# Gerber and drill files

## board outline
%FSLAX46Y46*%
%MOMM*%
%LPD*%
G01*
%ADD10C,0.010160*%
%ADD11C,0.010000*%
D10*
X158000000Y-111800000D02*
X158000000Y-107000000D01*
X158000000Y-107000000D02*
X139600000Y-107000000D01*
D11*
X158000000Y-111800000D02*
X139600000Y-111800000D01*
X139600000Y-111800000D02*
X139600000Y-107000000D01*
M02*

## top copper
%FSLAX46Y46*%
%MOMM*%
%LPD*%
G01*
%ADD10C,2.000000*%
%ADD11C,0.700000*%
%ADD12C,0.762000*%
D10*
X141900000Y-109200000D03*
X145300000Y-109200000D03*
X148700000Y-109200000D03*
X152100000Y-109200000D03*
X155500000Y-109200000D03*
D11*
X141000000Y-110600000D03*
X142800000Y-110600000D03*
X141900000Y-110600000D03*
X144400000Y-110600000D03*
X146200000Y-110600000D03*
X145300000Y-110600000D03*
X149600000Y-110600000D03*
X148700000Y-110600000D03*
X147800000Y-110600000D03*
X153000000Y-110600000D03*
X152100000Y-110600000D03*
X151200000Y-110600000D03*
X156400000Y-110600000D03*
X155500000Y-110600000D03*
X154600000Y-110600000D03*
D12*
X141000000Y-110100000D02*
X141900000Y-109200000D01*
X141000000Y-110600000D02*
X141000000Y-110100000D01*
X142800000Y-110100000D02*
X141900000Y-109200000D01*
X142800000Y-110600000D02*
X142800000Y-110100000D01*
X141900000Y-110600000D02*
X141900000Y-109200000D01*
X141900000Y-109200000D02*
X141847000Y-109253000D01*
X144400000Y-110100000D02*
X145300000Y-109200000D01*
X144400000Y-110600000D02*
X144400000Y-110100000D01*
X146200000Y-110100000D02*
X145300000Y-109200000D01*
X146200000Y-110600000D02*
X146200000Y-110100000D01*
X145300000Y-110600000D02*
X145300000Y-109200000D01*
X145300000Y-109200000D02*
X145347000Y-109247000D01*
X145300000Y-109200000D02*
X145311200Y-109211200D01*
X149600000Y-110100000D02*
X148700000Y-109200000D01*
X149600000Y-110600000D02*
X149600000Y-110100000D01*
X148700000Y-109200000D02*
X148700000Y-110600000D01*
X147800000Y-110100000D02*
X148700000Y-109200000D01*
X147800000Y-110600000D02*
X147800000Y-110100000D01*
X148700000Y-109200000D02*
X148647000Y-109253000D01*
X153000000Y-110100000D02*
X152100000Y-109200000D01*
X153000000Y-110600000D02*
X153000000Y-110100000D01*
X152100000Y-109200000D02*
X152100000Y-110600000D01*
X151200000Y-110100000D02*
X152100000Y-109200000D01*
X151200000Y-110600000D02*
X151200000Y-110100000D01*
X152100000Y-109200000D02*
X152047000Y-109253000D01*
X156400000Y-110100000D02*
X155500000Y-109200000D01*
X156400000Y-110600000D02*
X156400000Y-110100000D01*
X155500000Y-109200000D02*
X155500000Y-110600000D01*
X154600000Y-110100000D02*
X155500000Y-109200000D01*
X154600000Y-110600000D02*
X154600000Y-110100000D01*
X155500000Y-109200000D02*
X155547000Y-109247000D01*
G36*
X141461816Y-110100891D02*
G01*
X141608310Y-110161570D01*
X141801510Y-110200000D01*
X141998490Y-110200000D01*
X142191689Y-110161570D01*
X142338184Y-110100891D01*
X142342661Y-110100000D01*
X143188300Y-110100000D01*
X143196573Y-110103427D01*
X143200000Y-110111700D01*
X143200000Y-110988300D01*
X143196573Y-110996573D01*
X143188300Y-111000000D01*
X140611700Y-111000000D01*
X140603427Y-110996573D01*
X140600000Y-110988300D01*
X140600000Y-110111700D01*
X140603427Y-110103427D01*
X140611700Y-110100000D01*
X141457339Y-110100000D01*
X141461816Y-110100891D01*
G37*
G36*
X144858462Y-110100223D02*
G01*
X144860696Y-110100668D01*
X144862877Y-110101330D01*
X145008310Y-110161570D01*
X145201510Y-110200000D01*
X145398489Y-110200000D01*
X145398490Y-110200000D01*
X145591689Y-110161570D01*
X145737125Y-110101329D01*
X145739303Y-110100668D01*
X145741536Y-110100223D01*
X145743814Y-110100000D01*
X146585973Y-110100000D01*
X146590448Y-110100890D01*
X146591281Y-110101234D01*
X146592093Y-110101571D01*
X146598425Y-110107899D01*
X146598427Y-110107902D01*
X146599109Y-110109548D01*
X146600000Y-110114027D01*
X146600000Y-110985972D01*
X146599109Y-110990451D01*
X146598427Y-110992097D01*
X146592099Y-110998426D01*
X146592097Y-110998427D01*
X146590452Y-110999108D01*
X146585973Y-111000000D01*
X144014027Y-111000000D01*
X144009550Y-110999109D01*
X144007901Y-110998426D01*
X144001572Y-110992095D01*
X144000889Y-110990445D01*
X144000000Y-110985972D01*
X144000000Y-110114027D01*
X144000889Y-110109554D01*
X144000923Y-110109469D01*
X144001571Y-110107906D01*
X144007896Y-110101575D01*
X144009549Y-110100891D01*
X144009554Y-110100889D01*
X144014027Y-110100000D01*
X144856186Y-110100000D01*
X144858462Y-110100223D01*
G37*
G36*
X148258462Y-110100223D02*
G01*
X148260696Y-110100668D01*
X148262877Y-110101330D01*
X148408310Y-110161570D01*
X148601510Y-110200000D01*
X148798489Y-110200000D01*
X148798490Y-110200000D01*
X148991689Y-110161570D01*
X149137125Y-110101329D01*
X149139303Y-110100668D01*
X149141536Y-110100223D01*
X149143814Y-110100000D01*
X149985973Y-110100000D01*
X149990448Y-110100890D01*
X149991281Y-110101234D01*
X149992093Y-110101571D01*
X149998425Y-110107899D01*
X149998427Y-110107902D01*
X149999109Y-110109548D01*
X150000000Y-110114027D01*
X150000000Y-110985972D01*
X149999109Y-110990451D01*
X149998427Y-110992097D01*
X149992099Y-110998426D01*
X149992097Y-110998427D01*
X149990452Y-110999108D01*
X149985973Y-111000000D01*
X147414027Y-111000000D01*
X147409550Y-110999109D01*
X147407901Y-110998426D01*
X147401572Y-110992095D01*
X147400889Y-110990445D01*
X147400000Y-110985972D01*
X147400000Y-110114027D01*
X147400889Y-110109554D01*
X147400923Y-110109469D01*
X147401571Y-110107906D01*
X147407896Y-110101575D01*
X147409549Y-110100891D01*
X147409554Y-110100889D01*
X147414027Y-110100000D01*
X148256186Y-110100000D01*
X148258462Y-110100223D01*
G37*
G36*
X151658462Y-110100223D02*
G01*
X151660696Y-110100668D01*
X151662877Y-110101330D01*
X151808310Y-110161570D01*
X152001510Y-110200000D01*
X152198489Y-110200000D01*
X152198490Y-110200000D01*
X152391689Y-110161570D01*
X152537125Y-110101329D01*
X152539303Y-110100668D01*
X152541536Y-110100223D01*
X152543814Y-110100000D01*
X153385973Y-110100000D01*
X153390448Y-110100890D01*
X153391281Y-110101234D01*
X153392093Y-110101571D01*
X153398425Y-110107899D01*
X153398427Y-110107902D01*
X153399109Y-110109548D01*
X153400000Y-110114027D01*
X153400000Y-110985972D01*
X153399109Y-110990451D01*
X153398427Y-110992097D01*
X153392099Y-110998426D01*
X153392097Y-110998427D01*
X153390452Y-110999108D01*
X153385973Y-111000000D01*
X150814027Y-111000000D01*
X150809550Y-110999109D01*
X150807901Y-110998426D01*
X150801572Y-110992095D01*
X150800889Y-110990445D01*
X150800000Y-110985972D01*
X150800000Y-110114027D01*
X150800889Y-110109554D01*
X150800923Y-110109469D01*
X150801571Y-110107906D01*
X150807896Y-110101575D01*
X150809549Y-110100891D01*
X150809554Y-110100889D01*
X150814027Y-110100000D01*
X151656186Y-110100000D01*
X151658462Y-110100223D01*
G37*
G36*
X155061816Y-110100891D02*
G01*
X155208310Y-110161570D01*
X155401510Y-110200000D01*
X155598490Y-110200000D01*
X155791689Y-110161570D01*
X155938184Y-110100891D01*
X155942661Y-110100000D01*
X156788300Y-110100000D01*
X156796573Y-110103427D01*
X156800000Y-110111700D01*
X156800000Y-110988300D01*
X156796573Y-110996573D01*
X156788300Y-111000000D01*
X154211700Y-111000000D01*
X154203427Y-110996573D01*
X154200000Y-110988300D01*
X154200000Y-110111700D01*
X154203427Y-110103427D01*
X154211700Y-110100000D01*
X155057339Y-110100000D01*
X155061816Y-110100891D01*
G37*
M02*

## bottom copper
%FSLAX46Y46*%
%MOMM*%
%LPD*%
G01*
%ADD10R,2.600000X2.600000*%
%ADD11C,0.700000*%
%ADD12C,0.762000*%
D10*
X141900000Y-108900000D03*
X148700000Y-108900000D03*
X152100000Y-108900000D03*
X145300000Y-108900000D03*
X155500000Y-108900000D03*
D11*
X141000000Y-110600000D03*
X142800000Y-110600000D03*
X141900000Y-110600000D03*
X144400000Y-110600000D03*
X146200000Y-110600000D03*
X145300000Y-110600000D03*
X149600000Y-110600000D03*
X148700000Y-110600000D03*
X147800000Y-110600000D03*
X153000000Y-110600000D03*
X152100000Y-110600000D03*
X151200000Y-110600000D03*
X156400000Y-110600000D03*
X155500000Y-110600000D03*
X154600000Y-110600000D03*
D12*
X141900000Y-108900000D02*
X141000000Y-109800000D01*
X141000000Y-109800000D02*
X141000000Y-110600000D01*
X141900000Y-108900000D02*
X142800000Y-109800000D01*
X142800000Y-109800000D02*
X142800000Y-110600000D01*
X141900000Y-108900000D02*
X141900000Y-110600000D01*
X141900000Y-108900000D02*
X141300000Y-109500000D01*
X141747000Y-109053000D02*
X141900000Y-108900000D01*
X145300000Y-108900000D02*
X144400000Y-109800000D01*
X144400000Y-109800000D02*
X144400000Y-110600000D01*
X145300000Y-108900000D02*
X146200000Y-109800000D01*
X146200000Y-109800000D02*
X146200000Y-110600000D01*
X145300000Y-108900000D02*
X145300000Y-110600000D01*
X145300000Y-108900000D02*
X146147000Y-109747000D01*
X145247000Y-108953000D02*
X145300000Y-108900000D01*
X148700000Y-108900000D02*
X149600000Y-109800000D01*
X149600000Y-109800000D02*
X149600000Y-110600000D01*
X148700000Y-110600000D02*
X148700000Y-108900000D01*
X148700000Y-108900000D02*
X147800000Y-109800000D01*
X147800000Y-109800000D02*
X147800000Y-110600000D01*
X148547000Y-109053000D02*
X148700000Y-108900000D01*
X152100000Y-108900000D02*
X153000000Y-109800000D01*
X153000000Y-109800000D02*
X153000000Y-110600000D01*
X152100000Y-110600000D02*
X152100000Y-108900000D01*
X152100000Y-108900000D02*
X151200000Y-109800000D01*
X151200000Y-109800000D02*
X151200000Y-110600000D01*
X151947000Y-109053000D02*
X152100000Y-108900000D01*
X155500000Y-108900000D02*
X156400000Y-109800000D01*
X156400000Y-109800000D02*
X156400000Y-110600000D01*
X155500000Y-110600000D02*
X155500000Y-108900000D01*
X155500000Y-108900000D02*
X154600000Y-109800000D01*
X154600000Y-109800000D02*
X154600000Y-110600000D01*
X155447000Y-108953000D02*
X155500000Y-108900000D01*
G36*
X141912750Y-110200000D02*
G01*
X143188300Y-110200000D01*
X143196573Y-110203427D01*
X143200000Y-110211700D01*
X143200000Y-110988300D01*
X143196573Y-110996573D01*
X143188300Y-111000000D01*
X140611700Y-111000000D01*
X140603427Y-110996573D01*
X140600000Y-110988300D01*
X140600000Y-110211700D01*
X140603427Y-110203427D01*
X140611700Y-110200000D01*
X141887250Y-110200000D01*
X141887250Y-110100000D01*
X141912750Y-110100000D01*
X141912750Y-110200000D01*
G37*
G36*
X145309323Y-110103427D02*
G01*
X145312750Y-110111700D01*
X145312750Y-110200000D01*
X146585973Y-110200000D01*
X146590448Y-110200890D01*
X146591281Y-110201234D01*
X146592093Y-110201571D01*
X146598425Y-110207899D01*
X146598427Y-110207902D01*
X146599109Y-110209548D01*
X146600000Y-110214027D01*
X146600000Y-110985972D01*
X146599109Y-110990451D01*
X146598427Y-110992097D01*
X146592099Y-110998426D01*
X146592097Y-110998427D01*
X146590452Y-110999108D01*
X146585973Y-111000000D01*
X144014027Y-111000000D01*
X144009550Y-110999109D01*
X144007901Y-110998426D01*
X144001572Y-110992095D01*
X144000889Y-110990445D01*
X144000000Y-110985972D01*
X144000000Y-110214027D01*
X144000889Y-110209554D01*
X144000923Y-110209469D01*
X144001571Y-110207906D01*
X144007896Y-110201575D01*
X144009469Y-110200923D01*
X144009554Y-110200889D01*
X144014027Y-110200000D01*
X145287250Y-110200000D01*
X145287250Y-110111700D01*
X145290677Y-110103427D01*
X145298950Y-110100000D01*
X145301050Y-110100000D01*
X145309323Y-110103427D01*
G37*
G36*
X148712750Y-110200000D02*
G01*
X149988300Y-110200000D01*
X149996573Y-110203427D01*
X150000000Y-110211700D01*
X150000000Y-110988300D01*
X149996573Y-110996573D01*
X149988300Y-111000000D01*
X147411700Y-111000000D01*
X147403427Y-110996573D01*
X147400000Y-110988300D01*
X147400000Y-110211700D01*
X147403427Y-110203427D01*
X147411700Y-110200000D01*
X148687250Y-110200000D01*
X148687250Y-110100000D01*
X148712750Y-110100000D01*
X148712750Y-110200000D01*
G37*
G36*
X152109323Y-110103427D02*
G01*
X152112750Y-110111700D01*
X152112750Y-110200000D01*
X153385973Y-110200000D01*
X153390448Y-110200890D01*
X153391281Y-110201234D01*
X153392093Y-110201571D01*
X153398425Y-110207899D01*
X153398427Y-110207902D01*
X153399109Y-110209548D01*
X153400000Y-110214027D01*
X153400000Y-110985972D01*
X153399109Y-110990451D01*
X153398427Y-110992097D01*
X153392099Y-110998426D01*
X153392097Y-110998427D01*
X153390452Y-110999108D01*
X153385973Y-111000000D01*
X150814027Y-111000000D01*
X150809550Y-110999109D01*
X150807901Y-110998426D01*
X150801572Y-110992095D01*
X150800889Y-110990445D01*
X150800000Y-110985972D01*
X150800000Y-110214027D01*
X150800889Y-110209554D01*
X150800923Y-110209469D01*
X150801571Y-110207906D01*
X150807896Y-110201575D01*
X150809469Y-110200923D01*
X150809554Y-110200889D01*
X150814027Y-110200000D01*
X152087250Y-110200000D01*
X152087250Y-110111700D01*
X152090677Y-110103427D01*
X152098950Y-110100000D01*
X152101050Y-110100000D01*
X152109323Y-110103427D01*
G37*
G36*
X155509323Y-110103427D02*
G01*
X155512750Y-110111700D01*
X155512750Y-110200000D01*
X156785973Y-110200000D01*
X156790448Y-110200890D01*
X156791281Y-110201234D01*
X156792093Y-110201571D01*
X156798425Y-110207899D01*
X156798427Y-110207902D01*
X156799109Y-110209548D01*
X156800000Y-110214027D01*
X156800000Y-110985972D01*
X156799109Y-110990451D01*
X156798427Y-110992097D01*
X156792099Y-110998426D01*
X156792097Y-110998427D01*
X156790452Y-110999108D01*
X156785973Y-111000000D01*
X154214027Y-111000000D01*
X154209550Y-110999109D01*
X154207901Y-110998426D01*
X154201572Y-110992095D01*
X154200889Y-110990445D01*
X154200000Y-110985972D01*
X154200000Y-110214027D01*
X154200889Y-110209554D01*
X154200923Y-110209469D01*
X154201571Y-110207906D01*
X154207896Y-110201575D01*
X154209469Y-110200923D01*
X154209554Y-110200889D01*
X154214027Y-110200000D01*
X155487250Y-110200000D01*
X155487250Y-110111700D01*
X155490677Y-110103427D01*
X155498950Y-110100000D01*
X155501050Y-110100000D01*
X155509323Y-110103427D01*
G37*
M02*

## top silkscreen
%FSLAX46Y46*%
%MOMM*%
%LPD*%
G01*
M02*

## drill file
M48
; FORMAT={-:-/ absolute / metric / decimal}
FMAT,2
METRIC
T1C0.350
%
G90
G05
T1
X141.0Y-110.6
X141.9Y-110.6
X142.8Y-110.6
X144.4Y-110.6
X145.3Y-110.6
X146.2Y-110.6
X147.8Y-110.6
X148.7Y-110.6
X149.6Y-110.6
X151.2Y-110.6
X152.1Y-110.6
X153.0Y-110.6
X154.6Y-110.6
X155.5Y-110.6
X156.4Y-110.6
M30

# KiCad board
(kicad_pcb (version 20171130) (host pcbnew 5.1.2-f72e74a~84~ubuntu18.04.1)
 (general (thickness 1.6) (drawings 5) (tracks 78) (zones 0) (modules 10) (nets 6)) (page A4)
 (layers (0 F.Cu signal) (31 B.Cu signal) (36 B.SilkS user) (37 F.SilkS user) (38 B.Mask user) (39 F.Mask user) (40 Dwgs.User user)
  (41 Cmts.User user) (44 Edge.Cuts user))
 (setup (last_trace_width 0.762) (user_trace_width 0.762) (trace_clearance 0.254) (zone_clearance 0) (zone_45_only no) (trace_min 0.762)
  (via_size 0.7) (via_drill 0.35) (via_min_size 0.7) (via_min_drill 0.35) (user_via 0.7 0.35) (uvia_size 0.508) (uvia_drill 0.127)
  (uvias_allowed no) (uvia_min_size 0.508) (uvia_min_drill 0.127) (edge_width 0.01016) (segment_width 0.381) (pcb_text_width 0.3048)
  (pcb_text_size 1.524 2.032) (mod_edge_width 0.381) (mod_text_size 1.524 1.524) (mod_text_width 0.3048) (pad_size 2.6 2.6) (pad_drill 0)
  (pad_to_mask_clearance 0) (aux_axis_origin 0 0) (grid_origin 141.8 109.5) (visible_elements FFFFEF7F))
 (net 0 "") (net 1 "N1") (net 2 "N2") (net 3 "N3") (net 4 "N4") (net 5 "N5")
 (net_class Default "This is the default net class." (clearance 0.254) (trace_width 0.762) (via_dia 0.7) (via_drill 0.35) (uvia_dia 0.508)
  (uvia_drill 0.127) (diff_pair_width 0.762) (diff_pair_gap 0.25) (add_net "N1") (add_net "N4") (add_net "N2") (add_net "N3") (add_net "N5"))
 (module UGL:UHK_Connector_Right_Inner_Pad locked (layer B.Cu) (at 146.31 108.9)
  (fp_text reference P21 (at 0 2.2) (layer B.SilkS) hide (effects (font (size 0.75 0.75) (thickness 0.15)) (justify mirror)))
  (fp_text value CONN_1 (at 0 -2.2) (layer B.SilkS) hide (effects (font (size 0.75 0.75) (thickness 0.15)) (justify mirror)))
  (pad 1 smd rect (at -4.41 0) (size 2.6 2.6) (layers B.Cu B.Mask) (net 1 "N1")))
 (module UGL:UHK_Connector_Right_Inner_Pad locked (layer B.Cu) (at 151.15 108.9)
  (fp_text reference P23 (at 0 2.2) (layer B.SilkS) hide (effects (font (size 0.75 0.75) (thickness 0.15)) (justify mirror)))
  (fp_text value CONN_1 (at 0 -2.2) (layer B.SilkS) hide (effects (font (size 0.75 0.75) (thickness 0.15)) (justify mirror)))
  (pad 1 smd rect (at -2.45 0) (size 2.6 2.6) (layers B.Cu B.Mask) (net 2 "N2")))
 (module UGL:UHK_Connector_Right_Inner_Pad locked (layer B.Cu) (at 153.57 108.9)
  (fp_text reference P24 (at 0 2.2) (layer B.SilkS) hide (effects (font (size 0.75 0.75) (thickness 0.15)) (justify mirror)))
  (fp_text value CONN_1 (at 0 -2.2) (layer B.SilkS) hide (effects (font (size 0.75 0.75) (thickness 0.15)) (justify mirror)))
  (pad 1 smd rect (at -1.47 0) (size 2.6 2.6) (layers B.Cu B.Mask) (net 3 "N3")))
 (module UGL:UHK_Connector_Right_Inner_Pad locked (layer B.Cu) (at 148.73 108.9)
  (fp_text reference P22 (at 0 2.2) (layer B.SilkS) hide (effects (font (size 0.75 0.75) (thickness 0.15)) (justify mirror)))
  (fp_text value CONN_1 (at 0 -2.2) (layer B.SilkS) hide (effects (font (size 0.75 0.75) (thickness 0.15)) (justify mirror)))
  (pad 1 smd rect (at -3.43 0) (size 2.6 2.6) (layers B.Cu B.Mask) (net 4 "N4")))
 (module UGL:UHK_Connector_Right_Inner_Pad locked (layer B.Cu) (at 155.99 108.9)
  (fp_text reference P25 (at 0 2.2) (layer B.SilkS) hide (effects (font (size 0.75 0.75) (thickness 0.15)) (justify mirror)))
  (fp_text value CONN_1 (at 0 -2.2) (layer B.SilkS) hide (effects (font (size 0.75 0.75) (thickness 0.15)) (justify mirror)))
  (pad 1 smd rect (at -0.49 0) (size 2.6 2.6) (layers B.Cu B.Mask) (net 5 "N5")))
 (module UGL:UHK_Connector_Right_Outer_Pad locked (layer F.Cu) (at 141.9 109.2)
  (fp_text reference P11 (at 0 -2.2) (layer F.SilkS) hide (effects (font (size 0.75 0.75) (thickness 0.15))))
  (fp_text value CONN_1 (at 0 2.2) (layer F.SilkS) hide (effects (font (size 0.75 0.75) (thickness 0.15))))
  (pad 1 smd circle (at 0 0) (size 2 2) (layers F.Cu F.Mask) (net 1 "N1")))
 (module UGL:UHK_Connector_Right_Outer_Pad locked (layer F.Cu) (at 145.3 109.2)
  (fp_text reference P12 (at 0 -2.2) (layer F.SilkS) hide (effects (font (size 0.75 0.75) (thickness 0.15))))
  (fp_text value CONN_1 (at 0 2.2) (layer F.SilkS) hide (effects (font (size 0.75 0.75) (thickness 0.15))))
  (pad 1 smd circle (at 0 0) (size 2 2) (layers F.Cu F.Mask) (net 4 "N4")))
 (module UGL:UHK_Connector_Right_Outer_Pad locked (layer F.Cu) (at 148.7 109.2)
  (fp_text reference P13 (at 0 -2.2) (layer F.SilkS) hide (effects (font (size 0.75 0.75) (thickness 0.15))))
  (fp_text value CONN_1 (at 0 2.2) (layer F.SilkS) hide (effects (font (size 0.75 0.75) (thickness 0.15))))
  (pad 1 smd circle (at 0 0) (size 2 2) (layers F.Cu F.Mask) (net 2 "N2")))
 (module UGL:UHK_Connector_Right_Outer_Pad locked (layer F.Cu) (at 152.1 109.2)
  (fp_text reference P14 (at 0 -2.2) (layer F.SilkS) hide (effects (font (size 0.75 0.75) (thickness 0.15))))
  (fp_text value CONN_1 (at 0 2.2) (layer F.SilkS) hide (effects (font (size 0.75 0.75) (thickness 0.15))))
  (pad 1 smd circle (at 0 0) (size 2 2) (layers F.Cu F.Mask) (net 3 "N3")))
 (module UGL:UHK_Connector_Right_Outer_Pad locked (layer F.Cu) (at 155.5 109.2)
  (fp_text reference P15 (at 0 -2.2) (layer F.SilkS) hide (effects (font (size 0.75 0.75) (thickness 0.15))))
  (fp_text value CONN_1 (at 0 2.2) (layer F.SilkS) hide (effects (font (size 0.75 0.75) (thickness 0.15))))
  (pad 1 smd circle (at 0 0) (size 2 2) (layers F.Cu F.Mask) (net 5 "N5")))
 (gr_line (start 158 111.8) (end 158 107) (layer Edge.Cuts) (width 0.01016))
 (gr_line (start 158 107) (end 139.6 107) (layer Edge.Cuts) (width 0.01016))
 (gr_line (start 158 111.8) (end 139.6 111.8) (angle 90) (layer Edge.Cuts) (width 0.01))
 (gr_line (start 139.6 111.8) (end 139.6 107) (angle 90) (layer Edge.Cuts) (width 0.01))
 (segment (start 141.9 108.9) (end 141 109.8) (width 0.762) (layer B.Cu) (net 1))
 (segment (start 141 109.8) (end 141 110.6) (width 0.762) (layer B.Cu) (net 1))
 (segment (start 141 110.1) (end 141.9 109.2) (width 0.762) (layer F.Cu) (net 1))
 (segment (start 141 110.6) (end 141 110.1) (width 0.762) (layer F.Cu) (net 1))
 (via (at 141 110.6) (size 0.7) (drill 0.35) (layers F.Cu B.Cu) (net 1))
 (segment (start 141.9 108.9) (end 142.8 109.8) (width 0.762) (layer B.Cu) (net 1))
 (segment (start 142.8 109.8) (end 142.8 110.6) (width 0.762) (layer B.Cu) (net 1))
 (segment (start 142.8 110.1) (end 141.9 109.2) (width 0.762) (layer F.Cu) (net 1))
 (segment (start 142.8 110.6) (end 142.8 110.1) (width 0.762) (layer F.Cu) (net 1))
 (via (at 142.8 110.6) (size 0.7) (drill 0.35) (layers F.Cu B.Cu) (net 1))
 (segment (start 141.9 108.9) (end 141.9 110.6) (width 0.762) (layer B.Cu) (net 1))
 (segment (start 141.9 110.6) (end 141.9 109.2) (width 0.762) (layer F.Cu) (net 1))
 (via (at 141.9 110.6) (size 0.7) (drill 0.35) (layers F.Cu B.Cu) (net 1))
 (segment (start 141.9 108.9) (end 141.3 109.5) (width 0.762) (layer B.Cu) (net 1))
 (segment (start 141.9 109.2) (end 141.847 109.253) (width 0.762) (layer F.Cu) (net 1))
 (segment (start 141.747 109.053) (end 141.9 108.9) (width 0.762) (layer B.Cu) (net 1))
 (segment (start 145.3 108.9) (end 144.4 109.8) (width 0.762) (layer B.Cu) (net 4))
 (segment (start 144.4 109.8) (end 144.4 110.6) (width 0.762) (layer B.Cu) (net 4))
 (segment (start 144.4 110.1) (end 145.3 109.2) (width 0.762) (layer F.Cu) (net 4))
 (segment (start 144.4 110.6) (end 144.4 110.1) (width 0.762) (layer F.Cu) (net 4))
 (via (at 144.4 110.6) (size 0.7) (drill 0.35) (layers F.Cu B.Cu) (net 4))
 (segment (start 145.3 108.9) (end 146.2 109.8) (width 0.762) (layer B.Cu) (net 4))
 (segment (start 146.2 109.8) (end 146.2 110.6) (width 0.762) (layer B.Cu) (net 4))
 (segment (start 146.2 110.1) (end 145.3 109.2) (width 0.762) (layer F.Cu) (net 4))
 (segment (start 146.2 110.6) (end 146.2 110.1) (width 0.762) (layer F.Cu) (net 4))
 (via (at 146.2 110.6) (size 0.7) (drill 0.35) (layers F.Cu B.Cu) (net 4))
 (segment (start 145.3 108.9) (end 145.3 110.6) (width 0.762) (layer B.Cu) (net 4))
 (segment (start 145.3 110.6) (end 145.3 109.2) (width 0.762) (layer F.Cu) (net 4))
 (via (at 145.3 110.6) (size 0.7) (drill 0.35) (layers F.Cu B.Cu) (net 4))
 (segment (start 145.3 108.9) (end 146.147 109.747) (width 0.762) (layer B.Cu) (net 4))
 (segment (start 145.3 109.2) (end 145.347 109.247) (width 0.762) (layer F.Cu) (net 4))
 (segment (start 145.247 108.953) (end 145.3 108.9) (width 0.762) (layer B.Cu) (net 4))
 (segment (start 145.3 109.2) (end 145.3112 109.2112) (width 0.762) (layer F.Cu) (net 4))
 (segment (start 148.7 108.9) (end 149.6 109.8) (width 0.762) (layer B.Cu) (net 2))
 (segment (start 149.6 109.8) (end 149.6 110.6) (width 0.762) (layer B.Cu) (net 2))
 (segment (start 149.6 110.1) (end 148.7 109.2) (width 0.762) (layer F.Cu) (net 2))
 (segment (start 149.6 110.6) (end 149.6 110.1) (width 0.762) (layer F.Cu) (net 2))
 (via (at 149.6 110.6) (size 0.7) (drill 0.35) (layers F.Cu B.Cu) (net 2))
 (segment (start 148.7 109.2) (end 148.7 110.6) (width 0.762) (layer F.Cu) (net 2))
 (segment (start 148.7 110.6) (end 148.7 108.9) (width 0.762) (layer B.Cu) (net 2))
 (via (at 148.7 110.6) (size 0.7) (drill 0.35) (layers F.Cu B.Cu) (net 2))
 (segment (start 148.7 108.9) (end 147.8 109.8) (width 0.762) (layer B.Cu) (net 2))
 (segment (start 147.8 109.8) (end 147.8 110.6) (width 0.762) (layer B.Cu) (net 2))
 (segment (start 147.8 110.1) (end 148.7 109.2) (width 0.762) (layer F.Cu) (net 2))
 (segment (start 147.8 110.6) (end 147.8 110.1) (width 0.762) (layer F.Cu) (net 2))
 (via (at 147.8 110.6) (size 0.7) (drill 0.35) (layers F.Cu B.Cu) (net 2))
 (segment (start 148.7 109.2) (end 148.647 109.253) (width 0.762) (layer F.Cu) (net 2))
 (segment (start 148.547 109.053) (end 148.7 108.9) (width 0.762) (layer B.Cu) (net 2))
 (segment (start 152.1 108.9) (end 153 109.8) (width 0.762) (layer B.Cu) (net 3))
 (segment (start 153 109.8) (end 153 110.6) (width 0.762) (layer B.Cu) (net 3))
 (segment (start 153 110.1) (end 152.1 109.2) (width 0.762) (layer F.Cu) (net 3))
 (segment (start 153 110.6) (end 153 110.1) (width 0.762) (layer F.Cu) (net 3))
 (via (at 153 110.6) (size 0.7) (drill 0.35) (layers F.Cu B.Cu) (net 3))
 (segment (start 152.1 109.2) (end 152.1 110.6) (width 0.762) (layer F.Cu) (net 3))
 (segment (start 152.1 110.6) (end 152.1 108.9) (width 0.762) (layer B.Cu) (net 3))
 (via (at 152.1 110.6) (size 0.7) (drill 0.35) (layers F.Cu B.Cu) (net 3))
 (segment (start 152.1 108.9) (end 151.2 109.8) (width 0.762) (layer B.Cu) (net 3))
 (segment (start 151.2 109.8) (end 151.2 110.6) (width 0.762) (layer B.Cu) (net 3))
 (segment (start 151.2 110.1) (end 152.1 109.2) (width 0.762) (layer F.Cu) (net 3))
 (segment (start 151.2 110.6) (end 151.2 110.1) (width 0.762) (layer F.Cu) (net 3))
 (via (at 151.2 110.6) (size 0.7) (drill 0.35) (layers F.Cu B.Cu) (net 3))
 (segment (start 152.1 109.2) (end 152.047 109.253) (width 0.762) (layer F.Cu) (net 3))
 (segment (start 151.947 109.053) (end 152.1 108.9) (width 0.762) (layer B.Cu) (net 3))
 (segment (start 155.5 108.9) (end 156.4 109.8) (width 0.762) (layer B.Cu) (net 5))
 (segment (start 156.4 109.8) (end 156.4 110.6) (width 0.762) (layer B.Cu) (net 5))
 (segment (start 156.4 110.1) (end 155.5 109.2) (width 0.762) (layer F.Cu) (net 5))
 (segment (start 156.4 110.6) (end 156.4 110.1) (width 0.762) (layer F.Cu) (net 5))
 (via (at 156.4 110.6) (size 0.7) (drill 0.35) (layers F.Cu B.Cu) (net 5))
 (segment (start 155.5 109.2) (end 155.5 110.6) (width 0.762) (layer F.Cu) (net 5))
 (segment (start 155.5 110.6) (end 155.5 108.9) (width 0.762) (layer B.Cu) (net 5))
 (via (at 155.5 110.6) (size 0.7) (drill 0.35) (layers F.Cu B.Cu) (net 5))
 (segment (start 155.5 108.9) (end 154.6 109.8) (width 0.762) (layer B.Cu) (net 5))
 (segment (start 154.6 109.8) (end 154.6 110.6) (width 0.762) (layer B.Cu) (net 5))
 (segment (start 154.6 110.1) (end 155.5 109.2) (width 0.762) (layer F.Cu) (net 5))
 (segment (start 154.6 110.6) (end 154.6 110.1) (width 0.762) (layer F.Cu) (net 5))
 (via (at 154.6 110.6) (size 0.7) (drill 0.35) (layers F.Cu B.Cu) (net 5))
 (segment (start 155.5 109.2) (end 155.547 109.247) (width 0.762) (layer F.Cu) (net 5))
 (segment (start 155.447 108.953) (end 155.5 108.9) (width 0.762) (layer B.Cu) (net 5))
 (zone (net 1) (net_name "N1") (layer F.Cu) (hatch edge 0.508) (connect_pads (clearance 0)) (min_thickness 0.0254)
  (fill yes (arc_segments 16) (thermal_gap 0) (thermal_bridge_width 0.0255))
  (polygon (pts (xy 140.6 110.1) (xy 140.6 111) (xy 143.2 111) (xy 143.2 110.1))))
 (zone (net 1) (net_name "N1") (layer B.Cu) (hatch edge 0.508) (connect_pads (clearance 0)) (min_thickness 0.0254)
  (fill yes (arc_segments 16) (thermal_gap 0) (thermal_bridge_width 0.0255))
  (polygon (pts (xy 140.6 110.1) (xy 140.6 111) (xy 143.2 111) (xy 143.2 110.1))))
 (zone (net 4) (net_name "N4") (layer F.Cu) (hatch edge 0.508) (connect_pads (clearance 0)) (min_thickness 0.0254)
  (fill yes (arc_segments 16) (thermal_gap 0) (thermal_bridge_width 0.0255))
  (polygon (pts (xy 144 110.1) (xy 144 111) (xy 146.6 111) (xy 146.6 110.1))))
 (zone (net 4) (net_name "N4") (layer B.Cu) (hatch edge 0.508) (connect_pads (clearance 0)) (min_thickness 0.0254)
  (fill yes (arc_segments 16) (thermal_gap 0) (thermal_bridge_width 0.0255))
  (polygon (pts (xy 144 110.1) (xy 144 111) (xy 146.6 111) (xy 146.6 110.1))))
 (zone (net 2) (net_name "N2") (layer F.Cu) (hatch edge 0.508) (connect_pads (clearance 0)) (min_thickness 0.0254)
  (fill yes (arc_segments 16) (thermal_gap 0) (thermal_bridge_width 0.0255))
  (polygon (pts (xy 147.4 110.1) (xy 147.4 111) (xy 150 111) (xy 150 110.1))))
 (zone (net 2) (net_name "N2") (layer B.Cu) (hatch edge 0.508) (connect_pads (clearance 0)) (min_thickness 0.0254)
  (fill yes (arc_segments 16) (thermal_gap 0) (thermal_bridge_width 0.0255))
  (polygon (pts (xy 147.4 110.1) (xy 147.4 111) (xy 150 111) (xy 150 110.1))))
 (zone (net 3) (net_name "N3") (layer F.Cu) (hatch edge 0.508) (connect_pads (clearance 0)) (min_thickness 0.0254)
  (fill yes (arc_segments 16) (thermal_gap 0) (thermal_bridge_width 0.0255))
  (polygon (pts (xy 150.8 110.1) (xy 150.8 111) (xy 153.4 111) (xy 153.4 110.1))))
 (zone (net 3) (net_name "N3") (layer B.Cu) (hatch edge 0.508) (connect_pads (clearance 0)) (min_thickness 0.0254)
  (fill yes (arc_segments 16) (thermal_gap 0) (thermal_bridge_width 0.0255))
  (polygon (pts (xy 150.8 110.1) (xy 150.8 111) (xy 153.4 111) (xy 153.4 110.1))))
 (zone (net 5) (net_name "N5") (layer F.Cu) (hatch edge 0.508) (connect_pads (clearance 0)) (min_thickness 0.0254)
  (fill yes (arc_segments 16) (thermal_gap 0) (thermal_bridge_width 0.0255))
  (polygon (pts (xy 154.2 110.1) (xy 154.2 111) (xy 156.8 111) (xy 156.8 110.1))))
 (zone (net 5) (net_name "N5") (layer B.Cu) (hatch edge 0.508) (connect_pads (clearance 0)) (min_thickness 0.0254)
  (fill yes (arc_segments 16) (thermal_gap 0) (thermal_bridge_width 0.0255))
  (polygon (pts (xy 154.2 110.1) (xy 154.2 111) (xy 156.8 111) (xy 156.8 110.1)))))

